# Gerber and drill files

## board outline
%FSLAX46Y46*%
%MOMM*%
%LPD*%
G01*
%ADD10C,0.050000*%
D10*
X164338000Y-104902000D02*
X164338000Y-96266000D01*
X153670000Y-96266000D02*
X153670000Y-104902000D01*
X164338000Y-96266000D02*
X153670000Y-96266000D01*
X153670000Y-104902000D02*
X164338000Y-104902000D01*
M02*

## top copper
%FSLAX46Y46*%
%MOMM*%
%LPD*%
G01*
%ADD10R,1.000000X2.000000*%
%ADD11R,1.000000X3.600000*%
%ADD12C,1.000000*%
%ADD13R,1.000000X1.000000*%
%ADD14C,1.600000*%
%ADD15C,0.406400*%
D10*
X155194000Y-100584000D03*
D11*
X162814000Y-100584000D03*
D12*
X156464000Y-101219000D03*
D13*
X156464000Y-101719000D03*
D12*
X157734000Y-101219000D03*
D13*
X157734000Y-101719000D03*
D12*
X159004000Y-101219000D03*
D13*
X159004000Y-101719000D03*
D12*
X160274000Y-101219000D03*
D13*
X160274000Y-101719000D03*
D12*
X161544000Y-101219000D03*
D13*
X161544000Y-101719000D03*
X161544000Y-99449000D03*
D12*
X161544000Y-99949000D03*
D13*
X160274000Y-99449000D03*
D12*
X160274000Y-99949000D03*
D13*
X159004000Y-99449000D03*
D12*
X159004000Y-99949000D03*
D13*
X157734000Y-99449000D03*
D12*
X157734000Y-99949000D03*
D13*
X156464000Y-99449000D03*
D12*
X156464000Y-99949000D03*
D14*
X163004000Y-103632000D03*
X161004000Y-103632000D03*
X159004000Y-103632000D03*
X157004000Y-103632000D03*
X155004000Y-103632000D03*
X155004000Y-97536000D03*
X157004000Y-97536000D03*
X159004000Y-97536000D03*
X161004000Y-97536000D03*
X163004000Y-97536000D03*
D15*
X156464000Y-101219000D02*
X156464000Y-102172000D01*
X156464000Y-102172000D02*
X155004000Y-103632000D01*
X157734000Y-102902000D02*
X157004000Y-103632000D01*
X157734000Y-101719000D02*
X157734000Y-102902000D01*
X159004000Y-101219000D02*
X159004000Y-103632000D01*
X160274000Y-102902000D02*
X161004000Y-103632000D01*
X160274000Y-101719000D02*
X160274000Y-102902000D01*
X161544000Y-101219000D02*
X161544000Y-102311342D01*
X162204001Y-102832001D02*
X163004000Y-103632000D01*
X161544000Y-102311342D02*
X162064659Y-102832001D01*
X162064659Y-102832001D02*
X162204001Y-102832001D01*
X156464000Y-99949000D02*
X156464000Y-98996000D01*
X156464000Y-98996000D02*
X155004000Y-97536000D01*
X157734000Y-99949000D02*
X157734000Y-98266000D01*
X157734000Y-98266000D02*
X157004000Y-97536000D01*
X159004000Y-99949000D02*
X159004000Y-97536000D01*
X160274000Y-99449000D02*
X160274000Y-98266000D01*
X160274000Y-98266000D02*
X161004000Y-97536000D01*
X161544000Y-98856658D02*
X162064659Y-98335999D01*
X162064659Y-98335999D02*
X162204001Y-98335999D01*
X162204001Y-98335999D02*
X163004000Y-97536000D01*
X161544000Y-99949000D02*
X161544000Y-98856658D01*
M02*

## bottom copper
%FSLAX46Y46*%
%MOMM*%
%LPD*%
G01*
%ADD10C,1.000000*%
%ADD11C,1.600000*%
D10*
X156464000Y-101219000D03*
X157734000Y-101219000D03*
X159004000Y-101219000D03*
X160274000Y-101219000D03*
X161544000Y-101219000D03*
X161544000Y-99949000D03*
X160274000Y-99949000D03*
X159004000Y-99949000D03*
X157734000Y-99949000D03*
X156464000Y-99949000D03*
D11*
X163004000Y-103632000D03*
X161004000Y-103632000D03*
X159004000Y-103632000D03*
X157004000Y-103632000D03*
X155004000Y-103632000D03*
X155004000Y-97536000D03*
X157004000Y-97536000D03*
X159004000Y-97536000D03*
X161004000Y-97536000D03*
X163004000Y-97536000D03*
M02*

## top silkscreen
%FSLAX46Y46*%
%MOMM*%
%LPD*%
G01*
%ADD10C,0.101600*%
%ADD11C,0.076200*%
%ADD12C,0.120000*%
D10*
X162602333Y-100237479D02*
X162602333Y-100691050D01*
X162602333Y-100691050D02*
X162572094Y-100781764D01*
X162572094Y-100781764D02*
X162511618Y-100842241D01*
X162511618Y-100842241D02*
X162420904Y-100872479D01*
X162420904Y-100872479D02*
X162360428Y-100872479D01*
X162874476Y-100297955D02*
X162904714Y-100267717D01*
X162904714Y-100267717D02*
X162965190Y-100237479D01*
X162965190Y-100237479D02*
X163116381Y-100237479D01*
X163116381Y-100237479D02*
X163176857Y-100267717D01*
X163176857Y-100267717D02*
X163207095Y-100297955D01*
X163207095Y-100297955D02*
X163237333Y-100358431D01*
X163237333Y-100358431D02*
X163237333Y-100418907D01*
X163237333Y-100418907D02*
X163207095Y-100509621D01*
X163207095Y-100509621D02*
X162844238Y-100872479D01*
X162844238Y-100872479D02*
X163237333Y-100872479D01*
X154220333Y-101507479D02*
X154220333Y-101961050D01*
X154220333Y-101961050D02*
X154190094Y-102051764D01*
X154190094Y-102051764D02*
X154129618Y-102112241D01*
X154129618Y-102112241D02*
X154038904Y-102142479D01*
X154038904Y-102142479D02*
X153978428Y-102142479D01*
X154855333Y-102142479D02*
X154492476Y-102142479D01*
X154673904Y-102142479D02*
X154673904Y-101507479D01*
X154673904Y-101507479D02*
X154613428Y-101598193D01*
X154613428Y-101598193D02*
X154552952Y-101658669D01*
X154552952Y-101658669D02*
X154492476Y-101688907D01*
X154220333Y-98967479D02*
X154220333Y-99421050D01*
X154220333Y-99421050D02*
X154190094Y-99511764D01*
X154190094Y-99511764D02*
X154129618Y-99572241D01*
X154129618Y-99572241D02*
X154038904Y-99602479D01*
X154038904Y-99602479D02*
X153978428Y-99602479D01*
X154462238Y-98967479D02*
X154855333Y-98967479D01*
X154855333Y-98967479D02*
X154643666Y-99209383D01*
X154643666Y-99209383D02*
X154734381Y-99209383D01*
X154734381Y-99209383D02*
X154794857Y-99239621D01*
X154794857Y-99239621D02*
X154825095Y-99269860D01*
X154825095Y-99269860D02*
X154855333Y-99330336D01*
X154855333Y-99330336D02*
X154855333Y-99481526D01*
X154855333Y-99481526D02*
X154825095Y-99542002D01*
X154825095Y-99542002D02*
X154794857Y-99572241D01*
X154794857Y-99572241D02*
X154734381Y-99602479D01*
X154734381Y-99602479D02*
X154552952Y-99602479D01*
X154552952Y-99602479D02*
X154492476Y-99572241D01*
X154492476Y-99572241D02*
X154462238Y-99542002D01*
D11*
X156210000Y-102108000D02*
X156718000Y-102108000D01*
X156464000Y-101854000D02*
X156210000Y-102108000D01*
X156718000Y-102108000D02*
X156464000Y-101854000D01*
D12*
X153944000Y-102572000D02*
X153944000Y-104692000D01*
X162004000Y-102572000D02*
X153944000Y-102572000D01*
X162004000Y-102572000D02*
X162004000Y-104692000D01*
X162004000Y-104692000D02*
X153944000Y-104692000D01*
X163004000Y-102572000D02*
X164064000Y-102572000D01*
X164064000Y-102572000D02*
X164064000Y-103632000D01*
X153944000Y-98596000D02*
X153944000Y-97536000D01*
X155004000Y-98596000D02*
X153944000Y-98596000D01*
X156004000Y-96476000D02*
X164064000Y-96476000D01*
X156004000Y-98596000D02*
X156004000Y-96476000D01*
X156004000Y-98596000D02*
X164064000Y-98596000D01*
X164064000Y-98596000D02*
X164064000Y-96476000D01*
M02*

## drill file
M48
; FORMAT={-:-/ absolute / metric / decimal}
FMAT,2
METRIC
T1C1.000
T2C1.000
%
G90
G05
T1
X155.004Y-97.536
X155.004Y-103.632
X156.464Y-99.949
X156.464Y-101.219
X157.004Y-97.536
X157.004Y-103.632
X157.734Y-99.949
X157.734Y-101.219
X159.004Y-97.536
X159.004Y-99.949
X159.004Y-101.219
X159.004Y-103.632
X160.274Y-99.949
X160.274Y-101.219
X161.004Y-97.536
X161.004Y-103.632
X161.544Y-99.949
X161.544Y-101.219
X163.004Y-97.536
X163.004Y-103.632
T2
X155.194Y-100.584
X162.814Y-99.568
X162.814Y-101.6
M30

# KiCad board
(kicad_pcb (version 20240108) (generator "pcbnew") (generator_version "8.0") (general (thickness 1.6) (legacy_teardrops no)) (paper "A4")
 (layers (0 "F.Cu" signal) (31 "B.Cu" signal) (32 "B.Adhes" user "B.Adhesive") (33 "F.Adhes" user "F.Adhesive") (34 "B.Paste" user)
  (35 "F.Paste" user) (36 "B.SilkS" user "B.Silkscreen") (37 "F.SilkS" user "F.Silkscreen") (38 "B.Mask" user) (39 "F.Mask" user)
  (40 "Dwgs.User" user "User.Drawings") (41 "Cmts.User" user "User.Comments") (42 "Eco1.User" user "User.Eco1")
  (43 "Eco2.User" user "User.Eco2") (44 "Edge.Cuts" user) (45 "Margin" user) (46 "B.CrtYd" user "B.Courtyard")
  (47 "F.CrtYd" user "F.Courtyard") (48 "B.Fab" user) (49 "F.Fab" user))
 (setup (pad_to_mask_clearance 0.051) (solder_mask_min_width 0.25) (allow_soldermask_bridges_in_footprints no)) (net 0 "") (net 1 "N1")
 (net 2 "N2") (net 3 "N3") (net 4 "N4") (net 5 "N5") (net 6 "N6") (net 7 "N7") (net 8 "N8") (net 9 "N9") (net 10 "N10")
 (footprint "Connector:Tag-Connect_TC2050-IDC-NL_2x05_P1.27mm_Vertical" (layer "F.Cu") (at 159.004 100.584)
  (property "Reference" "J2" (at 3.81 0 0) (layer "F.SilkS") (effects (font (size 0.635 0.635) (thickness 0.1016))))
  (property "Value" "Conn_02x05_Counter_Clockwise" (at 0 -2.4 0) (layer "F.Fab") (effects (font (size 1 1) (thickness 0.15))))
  (fp_line (start -2.794 1.524) (end -2.286 1.524) (stroke (width 0.0762) (type solid)) (layer "F.SilkS"))
  (fp_line (start -2.54 1.27) (end -2.794 1.524) (stroke (width 0.0762) (type solid)) (layer "F.SilkS"))
  (fp_line (start -2.286 1.524) (end -2.54 1.27) (stroke (width 0.0762) (type solid)) (layer "F.SilkS"))
  (pad "" np_thru_hole circle (at -3.81 0) (size 1 1) (drill 1) (layers "*.Cu" "*.Mask"))
  (pad "" smd rect (at -3.81 0) (size 1 2) (layers "F.Cu" "F.Paste" "F.Mask"))
  (pad "" np_thru_hole circle (at 3.81 -1.016) (size 1 1) (drill 1) (layers "*.Cu" "*.Mask"))
  (pad "" smd rect (at 3.81 0) (size 1 3.6) (layers "F.Cu" "F.Paste" "F.Mask"))
  (pad "" np_thru_hole circle (at 3.81 1.016) (size 1 1) (drill 1) (layers "*.Cu" "*.Mask"))
  (pad "1" thru_hole circle (at -2.54 0.635) (size 1 1) (drill 1) (layers "*.Cu" "*.Mask") (remove_unused_layers no) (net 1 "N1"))
  (pad "1" smd rect (at -2.54 1.135) (size 1 1) (layers "F.Cu" "F.Paste" "F.Mask") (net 1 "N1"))
  (pad "2" thru_hole circle (at -1.27 0.635) (size 1 1) (drill 1) (layers "*.Cu" "*.Mask") (remove_unused_layers no) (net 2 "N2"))
  (pad "2" smd rect (at -1.27 1.135) (size 1 1) (layers "F.Cu" "F.Paste" "F.Mask") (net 2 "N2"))
  (pad "3" thru_hole circle (at 0 0.635) (size 1 1) (drill 1) (layers "*.Cu" "*.Mask") (remove_unused_layers no) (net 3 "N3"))
  (pad "3" smd rect (at 0 1.135) (size 1 1) (layers "F.Cu" "F.Paste" "F.Mask") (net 3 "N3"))
  (pad "4" thru_hole circle (at 1.27 0.635) (size 1 1) (drill 1) (layers "*.Cu" "*.Mask") (remove_unused_layers no) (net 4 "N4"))
  (pad "4" smd rect (at 1.27 1.135) (size 1 1) (layers "F.Cu" "F.Paste" "F.Mask") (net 4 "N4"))
  (pad "5" thru_hole circle (at 2.54 0.635) (size 1 1) (drill 1) (layers "*.Cu" "*.Mask") (remove_unused_layers no) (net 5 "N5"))
  (pad "5" smd rect (at 2.54 1.135) (size 1 1) (layers "F.Cu" "F.Paste" "F.Mask") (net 5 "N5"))
  (pad "6" smd rect (at 2.54 -1.135) (size 1 1) (layers "F.Cu" "F.Paste" "F.Mask") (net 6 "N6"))
  (pad "6" thru_hole circle (at 2.54 -0.635) (size 1 1) (drill 1) (layers "*.Cu" "*.Mask") (remove_unused_layers no) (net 6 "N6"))
  (pad "7" smd rect (at 1.27 -1.135) (size 1 1) (layers "F.Cu" "F.Paste" "F.Mask") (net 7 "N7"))
  (pad "7" thru_hole circle (at 1.27 -0.635) (size 1 1) (drill 1) (layers "*.Cu" "*.Mask") (remove_unused_layers no) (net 7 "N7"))
  (pad "8" smd rect (at 0 -1.135) (size 1 1) (layers "F.Cu" "F.Paste" "F.Mask") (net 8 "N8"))
  (pad "8" thru_hole circle (at 0 -0.635) (size 1 1) (drill 1) (layers "*.Cu" "*.Mask") (remove_unused_layers no) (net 8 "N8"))
  (pad "9" smd rect (at -1.27 -1.135) (size 1 1) (layers "F.Cu" "F.Paste" "F.Mask") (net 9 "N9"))
  (pad "9" thru_hole circle (at -1.27 -0.635) (size 1 1) (drill 1) (layers "*.Cu" "*.Mask") (remove_unused_layers no) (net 9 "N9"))
  (pad "10" smd rect (at -2.54 -1.135) (size 1 1) (layers "F.Cu" "F.Paste" "F.Mask") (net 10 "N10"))
  (pad "10" thru_hole circle (at -2.54 -0.635) (size 1 1) (drill 1) (layers "*.Cu" "*.Mask") (remove_unused_layers no) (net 10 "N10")))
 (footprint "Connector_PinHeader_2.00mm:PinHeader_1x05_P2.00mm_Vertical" (layer "F.Cu") (at 163.004 103.632 -90)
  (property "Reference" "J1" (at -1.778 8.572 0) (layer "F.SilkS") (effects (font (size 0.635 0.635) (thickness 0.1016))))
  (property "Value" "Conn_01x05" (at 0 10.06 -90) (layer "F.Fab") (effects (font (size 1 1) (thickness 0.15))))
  (fp_line (start -1.06 9.06) (end 1.06 9.06) (stroke (width 0.12) (type solid)) (layer "F.SilkS"))
  (fp_line (start -1.06 1) (end -1.06 9.06) (stroke (width 0.12) (type solid)) (layer "F.SilkS"))
  (fp_line (start -1.06 1) (end 1.06 1) (stroke (width 0.12) (type solid)) (layer "F.SilkS"))
  (fp_line (start 1.06 1) (end 1.06 9.06) (stroke (width 0.12) (type solid)) (layer "F.SilkS"))
  (fp_line (start -1.06 0) (end -1.06 -1.06) (stroke (width 0.12) (type solid)) (layer "F.SilkS"))
  (fp_line (start -1.06 -1.06) (end 0 -1.06) (stroke (width 0.12) (type solid)) (layer "F.SilkS"))
  (pad "1" thru_hole circle (at 0 0 270) (size 1.6 1.6) (drill 1) (layers "*.Cu" "*.Mask") (remove_unused_layers no) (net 5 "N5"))
  (pad "2" thru_hole circle (at 0 2 270) (size 1.6 1.6) (drill 1) (layers "*.Cu" "*.Mask") (remove_unused_layers no) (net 4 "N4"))
  (pad "3" thru_hole circle (at 0 4 270) (size 1.6 1.6) (drill 1) (layers "*.Cu" "*.Mask") (remove_unused_layers no) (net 3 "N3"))
  (pad "4" thru_hole circle (at 0 6 270) (size 1.6 1.6) (drill 1) (layers "*.Cu" "*.Mask") (remove_unused_layers no) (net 2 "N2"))
  (pad "5" thru_hole circle (at 0 8 270) (size 1.6 1.6) (drill 1) (layers "*.Cu" "*.Mask") (remove_unused_layers no) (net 1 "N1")))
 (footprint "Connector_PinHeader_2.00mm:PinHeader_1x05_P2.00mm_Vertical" (layer "F.Cu") (at 155.004 97.536 90)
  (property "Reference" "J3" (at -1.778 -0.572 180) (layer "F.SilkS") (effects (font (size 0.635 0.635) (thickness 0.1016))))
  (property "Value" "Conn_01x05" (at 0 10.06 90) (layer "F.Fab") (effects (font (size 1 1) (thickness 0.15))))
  (fp_line (start -1.06 -1.06) (end 0 -1.06) (stroke (width 0.12) (type solid)) (layer "F.SilkS"))
  (fp_line (start -1.06 0) (end -1.06 -1.06) (stroke (width 0.12) (type solid)) (layer "F.SilkS"))
  (fp_line (start 1.06 1) (end 1.06 9.06) (stroke (width 0.12) (type solid)) (layer "F.SilkS"))
  (fp_line (start -1.06 1) (end 1.06 1) (stroke (width 0.12) (type solid)) (layer "F.SilkS"))
  (fp_line (start -1.06 1) (end -1.06 9.06) (stroke (width 0.12) (type solid)) (layer "F.SilkS"))
  (fp_line (start -1.06 9.06) (end 1.06 9.06) (stroke (width 0.12) (type solid)) (layer "F.SilkS"))
  (pad "1" thru_hole circle (at 0 0 90) (size 1.6 1.6) (drill 1) (layers "*.Cu" "*.Mask") (remove_unused_layers no) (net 10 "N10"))
  (pad "2" thru_hole circle (at 0 2 90) (size 1.6 1.6) (drill 1) (layers "*.Cu" "*.Mask") (remove_unused_layers no) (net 9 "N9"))
  (pad "3" thru_hole circle (at 0 4 90) (size 1.6 1.6) (drill 1) (layers "*.Cu" "*.Mask") (remove_unused_layers no) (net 8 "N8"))
  (pad "4" thru_hole circle (at 0 6 90) (size 1.6 1.6) (drill 1) (layers "*.Cu" "*.Mask") (remove_unused_layers no) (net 7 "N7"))
  (pad "5" thru_hole circle (at 0 8 90) (size 1.6 1.6) (drill 1) (layers "*.Cu" "*.Mask") (remove_unused_layers no) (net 6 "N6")))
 (gr_line (start 164.338 104.902) (end 164.338 96.266) (stroke (width 0.05) (type solid)) (layer "Edge.Cuts"))
 (gr_line (start 153.67 96.266) (end 153.67 104.902) (stroke (width 0.05) (type solid)) (layer "Edge.Cuts"))
 (gr_line (start 164.338 96.266) (end 153.67 96.266) (stroke (width 0.05) (type solid)) (layer "Edge.Cuts"))
 (gr_line (start 153.67 104.902) (end 164.338 104.902) (stroke (width 0.05) (type solid)) (layer "Edge.Cuts"))
 (segment (start 156.464 101.219) (end 156.464 102.172) (width 0.4064) (layer "F.Cu") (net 1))
 (segment (start 156.464 102.172) (end 155.004 103.632) (width 0.4064) (layer "F.Cu") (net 1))
 (segment (start 157.734 102.902) (end 157.004 103.632) (width 0.4064) (layer "F.Cu") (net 2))
 (segment (start 157.734 101.719) (end 157.734 102.902) (width 0.4064) (layer "F.Cu") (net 2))
 (segment (start 159.004 101.219) (end 159.004 103.632) (width 0.4064) (layer "F.Cu") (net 3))
 (segment (start 160.274 102.902) (end 161.004 103.632) (width 0.4064) (layer "F.Cu") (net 4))
 (segment (start 160.274 101.719) (end 160.274 102.902) (width 0.4064) (layer "F.Cu") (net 4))
 (segment (start 161.544 101.219) (end 161.544 102.311342) (width 0.4064) (layer "F.Cu") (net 5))
 (segment (start 162.204001 102.832001) (end 163.004 103.632) (width 0.4064) (layer "F.Cu") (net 5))
 (segment (start 161.544 102.311342) (end 162.064659 102.832001) (width 0.4064) (layer "F.Cu") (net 5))
 (segment (start 162.064659 102.832001) (end 162.204001 102.832001) (width 0.4064) (layer "F.Cu") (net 5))
 (segment (start 156.464 99.949) (end 156.464 98.996) (width 0.4064) (layer "F.Cu") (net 10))
 (segment (start 156.464 98.996) (end 155.004 97.536) (width 0.4064) (layer "F.Cu") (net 10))
 (segment (start 157.734 99.949) (end 157.734 98.266) (width 0.4064) (layer "F.Cu") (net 9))
 (segment (start 157.734 98.266) (end 157.004 97.536) (width 0.4064) (layer "F.Cu") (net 9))
 (segment (start 159.004 99.949) (end 159.004 97.536) (width 0.4064) (layer "F.Cu") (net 8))
 (segment (start 160.274 99.449) (end 160.274 98.266) (width 0.4064) (layer "F.Cu") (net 7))
 (segment (start 160.274 98.266) (end 161.004 97.536) (width 0.4064) (layer "F.Cu") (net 7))
 (segment (start 161.544 98.856658) (end 162.064659 98.335999) (width 0.4064) (layer "F.Cu") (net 6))
 (segment (start 162.064659 98.335999) (end 162.204001 98.335999) (width 0.4064) (layer "F.Cu") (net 6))
 (segment (start 162.204001 98.335999) (end 163.004 97.536) (width 0.4064) (layer "F.Cu") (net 6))
 (segment (start 161.544 99.949) (end 161.544 98.856658) (width 0.4064) (layer "F.Cu") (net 6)))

